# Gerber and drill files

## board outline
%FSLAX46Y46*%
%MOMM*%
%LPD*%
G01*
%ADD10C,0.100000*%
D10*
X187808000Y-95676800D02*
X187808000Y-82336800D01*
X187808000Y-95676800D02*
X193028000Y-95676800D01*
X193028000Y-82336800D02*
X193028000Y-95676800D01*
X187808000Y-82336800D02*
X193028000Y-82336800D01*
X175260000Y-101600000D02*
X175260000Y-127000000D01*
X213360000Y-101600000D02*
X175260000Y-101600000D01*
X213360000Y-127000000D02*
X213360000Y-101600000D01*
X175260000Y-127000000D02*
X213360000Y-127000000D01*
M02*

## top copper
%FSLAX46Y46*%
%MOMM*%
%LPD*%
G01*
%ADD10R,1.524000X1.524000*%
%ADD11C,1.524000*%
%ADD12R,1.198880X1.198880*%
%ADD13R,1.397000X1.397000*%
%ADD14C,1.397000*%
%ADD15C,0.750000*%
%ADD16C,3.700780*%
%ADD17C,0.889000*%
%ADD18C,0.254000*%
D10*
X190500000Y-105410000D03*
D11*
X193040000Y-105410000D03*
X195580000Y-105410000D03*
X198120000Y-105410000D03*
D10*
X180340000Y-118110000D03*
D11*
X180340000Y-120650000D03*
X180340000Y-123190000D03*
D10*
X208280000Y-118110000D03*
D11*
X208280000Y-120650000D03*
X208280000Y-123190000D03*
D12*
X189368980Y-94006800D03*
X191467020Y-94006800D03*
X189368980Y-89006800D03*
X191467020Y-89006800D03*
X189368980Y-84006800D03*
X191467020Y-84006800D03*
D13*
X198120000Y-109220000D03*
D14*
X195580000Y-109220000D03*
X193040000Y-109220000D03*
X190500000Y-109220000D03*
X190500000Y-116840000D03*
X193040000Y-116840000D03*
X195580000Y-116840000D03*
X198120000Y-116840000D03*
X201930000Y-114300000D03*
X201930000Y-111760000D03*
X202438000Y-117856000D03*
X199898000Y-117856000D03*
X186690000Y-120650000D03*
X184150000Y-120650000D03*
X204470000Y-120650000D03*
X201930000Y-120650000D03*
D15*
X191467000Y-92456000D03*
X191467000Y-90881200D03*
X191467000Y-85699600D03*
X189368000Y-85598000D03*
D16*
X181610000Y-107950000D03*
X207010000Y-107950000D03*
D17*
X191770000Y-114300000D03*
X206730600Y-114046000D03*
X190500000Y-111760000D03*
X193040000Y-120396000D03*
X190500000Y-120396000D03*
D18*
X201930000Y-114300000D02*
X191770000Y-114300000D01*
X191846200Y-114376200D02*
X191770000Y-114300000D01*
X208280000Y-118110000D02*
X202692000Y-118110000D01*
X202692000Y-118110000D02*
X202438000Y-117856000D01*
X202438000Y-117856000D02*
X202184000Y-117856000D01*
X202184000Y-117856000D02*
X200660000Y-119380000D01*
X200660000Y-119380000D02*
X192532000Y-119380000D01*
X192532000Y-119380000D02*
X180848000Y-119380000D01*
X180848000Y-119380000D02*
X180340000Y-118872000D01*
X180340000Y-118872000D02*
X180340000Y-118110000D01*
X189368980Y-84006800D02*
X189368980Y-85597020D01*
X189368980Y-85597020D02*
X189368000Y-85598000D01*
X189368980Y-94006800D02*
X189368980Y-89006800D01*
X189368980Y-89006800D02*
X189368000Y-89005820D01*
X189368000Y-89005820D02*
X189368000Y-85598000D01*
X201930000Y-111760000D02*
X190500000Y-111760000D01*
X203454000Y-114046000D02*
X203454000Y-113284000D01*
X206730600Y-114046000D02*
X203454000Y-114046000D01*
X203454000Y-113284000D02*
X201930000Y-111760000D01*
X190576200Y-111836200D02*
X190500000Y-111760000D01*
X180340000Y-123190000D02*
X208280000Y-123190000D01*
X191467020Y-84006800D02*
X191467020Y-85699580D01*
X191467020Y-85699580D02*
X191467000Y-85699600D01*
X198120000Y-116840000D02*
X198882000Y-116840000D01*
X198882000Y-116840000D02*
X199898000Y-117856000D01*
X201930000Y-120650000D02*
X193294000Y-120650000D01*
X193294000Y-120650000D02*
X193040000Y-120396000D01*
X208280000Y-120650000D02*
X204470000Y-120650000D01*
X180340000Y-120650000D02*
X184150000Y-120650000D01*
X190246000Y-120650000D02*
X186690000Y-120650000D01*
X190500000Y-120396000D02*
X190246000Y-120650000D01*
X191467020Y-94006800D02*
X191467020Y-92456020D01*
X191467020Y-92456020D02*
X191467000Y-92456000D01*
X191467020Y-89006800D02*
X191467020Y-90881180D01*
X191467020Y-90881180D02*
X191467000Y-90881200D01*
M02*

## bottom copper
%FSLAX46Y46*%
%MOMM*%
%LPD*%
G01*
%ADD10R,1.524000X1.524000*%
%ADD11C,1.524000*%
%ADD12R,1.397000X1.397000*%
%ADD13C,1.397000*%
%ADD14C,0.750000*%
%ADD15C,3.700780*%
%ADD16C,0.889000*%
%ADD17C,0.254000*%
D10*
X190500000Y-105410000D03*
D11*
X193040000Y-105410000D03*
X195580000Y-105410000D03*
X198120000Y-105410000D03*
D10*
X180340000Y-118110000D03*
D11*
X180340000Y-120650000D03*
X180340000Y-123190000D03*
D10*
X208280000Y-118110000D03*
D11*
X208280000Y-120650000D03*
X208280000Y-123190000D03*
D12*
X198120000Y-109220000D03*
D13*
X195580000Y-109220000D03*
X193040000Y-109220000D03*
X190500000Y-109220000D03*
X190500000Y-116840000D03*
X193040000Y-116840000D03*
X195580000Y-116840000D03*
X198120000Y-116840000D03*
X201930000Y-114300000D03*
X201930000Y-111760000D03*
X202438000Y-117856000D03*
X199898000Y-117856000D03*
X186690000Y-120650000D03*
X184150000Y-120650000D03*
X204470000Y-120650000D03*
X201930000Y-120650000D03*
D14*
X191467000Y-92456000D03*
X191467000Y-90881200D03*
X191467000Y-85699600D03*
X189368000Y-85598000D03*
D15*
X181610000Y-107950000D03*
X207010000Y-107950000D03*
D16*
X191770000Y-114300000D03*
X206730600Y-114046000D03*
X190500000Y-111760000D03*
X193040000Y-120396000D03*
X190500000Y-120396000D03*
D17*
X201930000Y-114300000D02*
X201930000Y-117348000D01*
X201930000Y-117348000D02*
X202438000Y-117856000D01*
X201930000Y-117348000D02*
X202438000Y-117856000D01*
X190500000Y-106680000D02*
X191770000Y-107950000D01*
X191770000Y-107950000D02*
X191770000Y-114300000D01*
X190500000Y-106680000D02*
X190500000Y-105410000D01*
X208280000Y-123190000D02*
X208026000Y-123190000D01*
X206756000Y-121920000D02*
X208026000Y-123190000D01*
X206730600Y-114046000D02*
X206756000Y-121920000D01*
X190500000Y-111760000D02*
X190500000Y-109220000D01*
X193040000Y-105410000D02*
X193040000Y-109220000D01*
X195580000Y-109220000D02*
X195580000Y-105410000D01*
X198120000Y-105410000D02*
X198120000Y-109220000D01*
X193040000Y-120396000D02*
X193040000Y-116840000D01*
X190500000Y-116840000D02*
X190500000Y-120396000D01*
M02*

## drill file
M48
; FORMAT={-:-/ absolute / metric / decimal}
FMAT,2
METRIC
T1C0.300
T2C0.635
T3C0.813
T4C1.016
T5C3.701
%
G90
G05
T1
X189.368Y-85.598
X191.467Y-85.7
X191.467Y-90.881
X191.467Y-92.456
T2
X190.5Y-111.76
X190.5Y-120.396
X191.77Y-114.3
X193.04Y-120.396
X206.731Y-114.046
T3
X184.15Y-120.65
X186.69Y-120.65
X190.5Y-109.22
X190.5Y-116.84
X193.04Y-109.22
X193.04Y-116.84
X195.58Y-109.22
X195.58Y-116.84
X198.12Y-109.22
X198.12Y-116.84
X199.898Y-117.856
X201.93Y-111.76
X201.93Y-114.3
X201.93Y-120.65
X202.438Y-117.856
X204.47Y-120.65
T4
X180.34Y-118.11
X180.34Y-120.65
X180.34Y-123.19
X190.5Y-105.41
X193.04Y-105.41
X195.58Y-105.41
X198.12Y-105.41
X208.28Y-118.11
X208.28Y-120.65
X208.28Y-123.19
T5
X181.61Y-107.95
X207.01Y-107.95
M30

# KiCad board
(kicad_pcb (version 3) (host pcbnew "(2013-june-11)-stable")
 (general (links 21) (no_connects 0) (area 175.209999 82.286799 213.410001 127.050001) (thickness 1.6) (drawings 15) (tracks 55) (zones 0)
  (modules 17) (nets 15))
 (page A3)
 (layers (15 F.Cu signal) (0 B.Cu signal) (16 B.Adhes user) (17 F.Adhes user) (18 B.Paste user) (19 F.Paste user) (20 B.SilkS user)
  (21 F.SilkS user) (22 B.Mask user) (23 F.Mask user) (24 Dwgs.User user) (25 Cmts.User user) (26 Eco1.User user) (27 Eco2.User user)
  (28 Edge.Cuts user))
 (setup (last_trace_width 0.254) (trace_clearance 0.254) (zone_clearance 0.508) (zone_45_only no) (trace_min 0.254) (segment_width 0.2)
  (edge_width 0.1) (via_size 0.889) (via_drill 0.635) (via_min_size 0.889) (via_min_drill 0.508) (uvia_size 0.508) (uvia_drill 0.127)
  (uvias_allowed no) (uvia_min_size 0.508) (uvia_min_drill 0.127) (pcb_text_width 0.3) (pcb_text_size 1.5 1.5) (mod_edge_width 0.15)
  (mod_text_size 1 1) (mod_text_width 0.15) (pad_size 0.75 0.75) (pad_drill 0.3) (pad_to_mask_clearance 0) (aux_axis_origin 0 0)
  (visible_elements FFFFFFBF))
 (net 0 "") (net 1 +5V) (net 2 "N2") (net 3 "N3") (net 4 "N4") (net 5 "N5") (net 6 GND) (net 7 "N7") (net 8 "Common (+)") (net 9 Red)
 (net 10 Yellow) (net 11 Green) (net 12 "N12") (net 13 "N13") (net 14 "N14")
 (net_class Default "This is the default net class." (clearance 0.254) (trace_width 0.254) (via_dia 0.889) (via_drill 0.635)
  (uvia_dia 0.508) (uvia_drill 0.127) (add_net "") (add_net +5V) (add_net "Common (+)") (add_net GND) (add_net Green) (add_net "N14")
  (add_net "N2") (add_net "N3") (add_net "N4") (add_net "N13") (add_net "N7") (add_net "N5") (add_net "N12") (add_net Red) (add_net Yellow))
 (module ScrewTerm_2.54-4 (layer F.Cu) (at 194.31 105.41)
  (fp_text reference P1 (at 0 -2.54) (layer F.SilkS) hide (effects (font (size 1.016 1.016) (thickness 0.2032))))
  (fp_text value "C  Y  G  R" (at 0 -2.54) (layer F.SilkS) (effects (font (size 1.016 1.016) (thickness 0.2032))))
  (pad 1 thru_hole rect (at -3.81 0) (size 1.524 1.524) (drill 1.016) (layers *.Cu *.Mask F.SilkS) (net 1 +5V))
  (pad 2 thru_hole circle (at -1.27 0) (size 1.524 1.524) (drill 1.016) (layers *.Cu *.Mask F.SilkS) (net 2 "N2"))
  (pad 3 thru_hole circle (at 1.27 0) (size 1.524 1.524) (drill 1.016) (layers *.Cu *.Mask F.SilkS) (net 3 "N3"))
  (pad 4 thru_hole circle (at 3.81 0) (size 1.524 1.524) (drill 1.016) (layers *.Cu *.Mask F.SilkS) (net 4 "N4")))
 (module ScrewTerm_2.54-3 (layer F.Cu) (at 180.34 120.65 270)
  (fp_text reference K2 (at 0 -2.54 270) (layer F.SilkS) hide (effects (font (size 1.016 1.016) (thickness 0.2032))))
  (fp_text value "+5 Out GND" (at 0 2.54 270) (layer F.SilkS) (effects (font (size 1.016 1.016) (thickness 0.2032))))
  (pad 1 thru_hole rect (at -2.54 0 270) (size 1.524 1.524) (drill 1.016) (layers *.Cu *.Mask F.SilkS) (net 1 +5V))
  (pad 2 thru_hole circle (at 0 0 270) (size 1.524 1.524) (drill 1.016) (layers *.Cu *.Mask F.SilkS) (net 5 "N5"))
  (pad 3 thru_hole circle (at 2.54 0 270) (size 1.524 1.524) (drill 1.016) (layers *.Cu *.Mask F.SilkS) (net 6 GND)))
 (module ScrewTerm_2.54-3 (layer F.Cu) (at 208.28 120.65 270)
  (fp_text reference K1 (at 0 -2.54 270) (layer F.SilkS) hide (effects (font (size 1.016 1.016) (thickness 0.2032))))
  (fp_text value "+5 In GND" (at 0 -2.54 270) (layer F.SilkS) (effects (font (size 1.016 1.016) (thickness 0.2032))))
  (pad 1 thru_hole rect (at -2.54 0 270) (size 1.524 1.524) (drill 1.016) (layers *.Cu *.Mask F.SilkS) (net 1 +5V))
  (pad 2 thru_hole circle (at 0 0 270) (size 1.524 1.524) (drill 1.016) (layers *.Cu *.Mask F.SilkS) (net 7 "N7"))
  (pad 3 thru_hole circle (at 2.54 0 270) (size 1.524 1.524) (drill 1.016) (layers *.Cu *.Mask F.SilkS) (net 6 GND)))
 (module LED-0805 (layer F.Cu) (at 190.418 94.0068)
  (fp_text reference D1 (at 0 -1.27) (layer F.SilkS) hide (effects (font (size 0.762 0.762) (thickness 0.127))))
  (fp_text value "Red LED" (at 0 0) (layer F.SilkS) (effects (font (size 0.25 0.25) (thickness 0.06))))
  (pad 1 smd rect (at -1.04902 0) (size 1.19888 1.19888) (layers F.Cu F.Paste F.Mask) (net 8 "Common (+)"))
  (pad 2 smd rect (at 1.04902 0) (size 1.19888 1.19888) (layers F.Cu F.Paste F.Mask) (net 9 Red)))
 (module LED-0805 (layer F.Cu) (at 190.418 89.0068)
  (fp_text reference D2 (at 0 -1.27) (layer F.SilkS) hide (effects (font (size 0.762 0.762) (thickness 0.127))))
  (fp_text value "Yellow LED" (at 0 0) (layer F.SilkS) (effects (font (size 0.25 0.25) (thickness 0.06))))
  (pad 1 smd rect (at -1.04902 0) (size 1.19888 1.19888) (layers F.Cu F.Paste F.Mask) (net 8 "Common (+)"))
  (pad 2 smd rect (at 1.04902 0) (size 1.19888 1.19888) (layers F.Cu F.Paste F.Mask) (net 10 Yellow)))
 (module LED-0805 (layer F.Cu) (at 190.418 84.0068)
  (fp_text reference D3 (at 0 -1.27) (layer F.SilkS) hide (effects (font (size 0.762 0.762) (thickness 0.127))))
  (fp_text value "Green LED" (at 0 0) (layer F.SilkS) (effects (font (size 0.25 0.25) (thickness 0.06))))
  (pad 1 smd rect (at -1.04902 0) (size 1.19888 1.19888) (layers F.Cu F.Paste F.Mask) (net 8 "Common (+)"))
  (pad 2 smd rect (at 1.04902 0) (size 1.19888 1.19888) (layers F.Cu F.Paste F.Mask) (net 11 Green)))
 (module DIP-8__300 (layer F.Cu) (at 194.31 113.03 180)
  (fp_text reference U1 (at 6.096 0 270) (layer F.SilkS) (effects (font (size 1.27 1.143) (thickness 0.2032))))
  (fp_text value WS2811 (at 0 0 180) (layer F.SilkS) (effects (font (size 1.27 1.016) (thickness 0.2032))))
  (pad 1 thru_hole rect (at -3.81 3.81 180) (size 1.397 1.397) (drill 0.8128) (layers *.Cu *.Mask F.SilkS) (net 4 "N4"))
  (pad 2 thru_hole circle (at -1.27 3.81 180) (size 1.397 1.397) (drill 0.8128) (layers *.Cu *.Mask F.SilkS) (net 3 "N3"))
  (pad 3 thru_hole circle (at 1.27 3.81 180) (size 1.397 1.397) (drill 0.8128) (layers *.Cu *.Mask F.SilkS) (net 2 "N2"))
  (pad 4 thru_hole circle (at 3.81 3.81 180) (size 1.397 1.397) (drill 0.8128) (layers *.Cu *.Mask F.SilkS) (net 6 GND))
  (pad 5 thru_hole circle (at 3.81 -3.81 180) (size 1.397 1.397) (drill 0.8128) (layers *.Cu *.Mask F.SilkS) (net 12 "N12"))
  (pad 6 thru_hole circle (at 1.27 -3.81 180) (size 1.397 1.397) (drill 0.8128) (layers *.Cu *.Mask F.SilkS) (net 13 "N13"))
  (pad 7 thru_hole circle (at -1.27 -3.81 180) (size 1.397 1.397) (drill 0.8128) (layers *.Cu *.Mask F.SilkS))
  (pad 8 thru_hole circle (at -3.81 -3.81 180) (size 1.397 1.397) (drill 0.8128) (layers *.Cu *.Mask F.SilkS) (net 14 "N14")))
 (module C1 (layer F.Cu) (at 201.93 113.03 90)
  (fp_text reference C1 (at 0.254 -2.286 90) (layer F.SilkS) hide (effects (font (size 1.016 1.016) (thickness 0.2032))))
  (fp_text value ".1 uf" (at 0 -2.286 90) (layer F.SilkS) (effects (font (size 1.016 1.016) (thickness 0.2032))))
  (pad 1 thru_hole circle (at -1.27 0 90) (size 1.397 1.397) (drill 0.8128) (layers *.Cu *.Mask F.SilkS) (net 1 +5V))
  (pad 2 thru_hole circle (at 1.27 0 90) (size 1.397 1.397) (drill 0.8128) (layers *.Cu *.Mask F.SilkS) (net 6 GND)))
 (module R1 (layer F.Cu) (at 201.168 117.856 180) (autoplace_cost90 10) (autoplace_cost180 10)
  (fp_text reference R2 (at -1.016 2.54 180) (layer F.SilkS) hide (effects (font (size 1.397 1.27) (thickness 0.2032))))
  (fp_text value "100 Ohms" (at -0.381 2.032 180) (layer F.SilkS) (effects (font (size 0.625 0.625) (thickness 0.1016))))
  (pad 1 thru_hole circle (at -1.27 0 180) (size 1.397 1.397) (drill 0.8128) (layers *.Cu *.Mask F.SilkS) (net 1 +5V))
  (pad 2 thru_hole circle (at 1.27 0 180) (size 1.397 1.397) (drill 0.8128) (layers *.Cu *.Mask F.SilkS) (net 14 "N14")))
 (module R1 (layer F.Cu) (at 185.42 120.65 180) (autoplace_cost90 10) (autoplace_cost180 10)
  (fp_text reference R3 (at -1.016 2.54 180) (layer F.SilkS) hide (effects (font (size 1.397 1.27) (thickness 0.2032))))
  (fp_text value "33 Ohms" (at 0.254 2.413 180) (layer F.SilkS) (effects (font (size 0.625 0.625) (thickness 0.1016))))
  (pad 1 thru_hole circle (at -1.27 0 180) (size 1.397 1.397) (drill 0.8128) (layers *.Cu *.Mask F.SilkS) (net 12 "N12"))
  (pad 2 thru_hole circle (at 1.27 0 180) (size 1.397 1.397) (drill 0.8128) (layers *.Cu *.Mask F.SilkS) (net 5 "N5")))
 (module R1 (layer F.Cu) (at 203.2 120.65 180) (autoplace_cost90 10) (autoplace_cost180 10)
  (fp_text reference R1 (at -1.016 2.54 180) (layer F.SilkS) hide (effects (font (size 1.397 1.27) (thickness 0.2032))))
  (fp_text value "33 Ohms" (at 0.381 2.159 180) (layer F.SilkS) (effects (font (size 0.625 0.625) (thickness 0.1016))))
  (pad 1 thru_hole circle (at -1.27 0 180) (size 1.397 1.397) (drill 0.8128) (layers *.Cu *.Mask F.SilkS) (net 7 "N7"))
  (pad 2 thru_hole circle (at 1.27 0 180) (size 1.397 1.397) (drill 0.8128) (layers *.Cu *.Mask F.SilkS) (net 13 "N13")))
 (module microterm (layer F.Cu) (at 191.467 92.456)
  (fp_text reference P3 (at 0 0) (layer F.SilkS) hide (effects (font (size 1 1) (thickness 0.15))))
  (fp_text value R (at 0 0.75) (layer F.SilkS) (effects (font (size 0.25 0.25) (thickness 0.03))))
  (pad 1 thru_hole circle (at 0 0) (size 0.75 0.75) (drill 0.3) (layers *.Cu *.Mask F.SilkS) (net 9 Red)))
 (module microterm (layer F.Cu) (at 191.467 90.8812)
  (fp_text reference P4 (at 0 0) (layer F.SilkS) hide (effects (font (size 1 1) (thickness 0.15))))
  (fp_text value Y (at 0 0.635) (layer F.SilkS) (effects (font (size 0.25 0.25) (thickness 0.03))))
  (pad 1 thru_hole circle (at 0 0) (size 0.75 0.75) (drill 0.3) (layers *.Cu *.Mask F.SilkS) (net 10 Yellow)))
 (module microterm (layer F.Cu) (at 191.467 85.6996)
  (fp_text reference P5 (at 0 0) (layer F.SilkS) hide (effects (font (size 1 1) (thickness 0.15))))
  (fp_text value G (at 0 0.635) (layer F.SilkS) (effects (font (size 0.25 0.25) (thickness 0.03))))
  (pad 1 thru_hole circle (at 0 0) (size 0.75 0.75) (drill 0.3) (layers *.Cu *.Mask F.SilkS) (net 11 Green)))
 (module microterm (layer F.Cu) (at 189.368 85.598)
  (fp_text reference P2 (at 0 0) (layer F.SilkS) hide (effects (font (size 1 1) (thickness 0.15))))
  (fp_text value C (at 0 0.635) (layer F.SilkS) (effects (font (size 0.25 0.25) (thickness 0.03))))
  (pad 1 thru_hole circle (at 0 0) (size 0.75 0.75) (drill 0.3) (layers *.Cu *.Mask F.SilkS) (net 8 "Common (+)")))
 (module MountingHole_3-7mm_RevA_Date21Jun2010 (layer F.Cu) (at 181.61 107.95)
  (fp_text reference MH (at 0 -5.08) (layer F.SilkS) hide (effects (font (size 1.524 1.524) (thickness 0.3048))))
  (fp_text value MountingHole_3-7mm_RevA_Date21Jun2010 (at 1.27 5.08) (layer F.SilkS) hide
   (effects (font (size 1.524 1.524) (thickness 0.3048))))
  (pad 1 thru_hole circle (at 0 0) (size 3.70078 3.70078) (drill 3.70078) (layers)))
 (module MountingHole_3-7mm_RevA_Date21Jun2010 (layer F.Cu) (at 207.01 107.95)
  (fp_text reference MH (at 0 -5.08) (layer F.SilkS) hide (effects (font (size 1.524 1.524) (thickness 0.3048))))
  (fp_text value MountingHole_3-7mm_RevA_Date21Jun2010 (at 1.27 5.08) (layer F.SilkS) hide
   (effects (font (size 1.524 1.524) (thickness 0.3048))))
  (pad 1 thru_hole circle (at 0 0) (size 3.70078 3.70078) (drill 3.70078) (layers)))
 (gr_line (start 187.808 95.6768) (end 187.808 82.3368) (angle 90) (layer Edge.Cuts) (width 0.1))
 (gr_line (start 187.808 95.6768) (end 193.028 95.6768) (angle 90) (layer Edge.Cuts) (width 0.1))
 (gr_line (start 193.028 82.3368) (end 193.028 95.6768) (angle 90) (layer Edge.Cuts) (width 0.1))
 (gr_line (start 187.808 82.3368) (end 193.028 82.3368) (angle 90) (layer Edge.Cuts) (width 0.1))
 (gr_line (start 175.26 101.6) (end 175.26 127) (angle 90) (layer Edge.Cuts) (width 0.1))
 (gr_line (start 213.36 101.6) (end 175.26 101.6) (angle 90) (layer Edge.Cuts) (width 0.1))
 (gr_line (start 213.36 127) (end 213.36 101.6) (angle 90) (layer Edge.Cuts) (width 0.1))
 (gr_line (start 175.26 127) (end 213.36 127) (angle 90) (layer Edge.Cuts) (width 0.1))
 (segment (start 201.93 114.3) (end 201.93 117.348) (width 0.254) (layer B.Cu) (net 1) (status 400000))
 (segment (start 201.93 117.348) (end 202.438 117.856) (width 0.254) (layer B.Cu) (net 1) (status 800000))
 (segment (start 201.93 114.3) (end 191.77 114.3) (width 0.254) (layer F.Cu) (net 1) (status 400000))
 (segment (start 201.93 117.348) (end 202.438 117.856) (width 0.254) (layer B.Cu) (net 1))
 (segment (start 190.5 106.68) (end 191.77 107.95) (width 0.254) (layer B.Cu) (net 1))
 (segment (start 191.77 107.95) (end 191.77 114.3) (width 0.254) (layer B.Cu) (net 1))
 (via (at 191.77 114.3) (size 0.889) (layers F.Cu B.Cu) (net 1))
 (segment (start 190.5 106.68) (end 190.5 105.41) (width 0.254) (layer B.Cu) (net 1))
 (segment (start 191.8462 114.3762) (end 191.77 114.3) (width 0.254) (layer F.Cu) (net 1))
 (segment (start 208.28 118.11) (end 202.692 118.11) (width 0.254) (layer F.Cu) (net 1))
 (segment (start 202.692 118.11) (end 202.438 117.856) (width 0.254) (layer F.Cu) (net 1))
 (segment (start 202.438 117.856) (end 202.184 117.856) (width 0.254) (layer F.Cu) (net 1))
 (segment (start 202.184 117.856) (end 200.66 119.38) (width 0.254) (layer F.Cu) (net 1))
 (segment (start 200.66 119.38) (end 192.532 119.38) (width 0.254) (layer F.Cu) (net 1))
 (segment (start 192.532 119.38) (end 180.848 119.38) (width 0.254) (layer F.Cu) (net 1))
 (segment (start 180.848 119.38) (end 180.34 118.872) (width 0.254) (layer F.Cu) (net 1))
 (segment (start 180.34 118.872) (end 180.34 118.11) (width 0.254) (layer F.Cu) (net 1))
 (segment (start 189.36898 84.0068) (end 189.36898 85.59702) (width 0.254) (layer F.Cu) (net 8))
 (segment (start 189.36898 85.59702) (end 189.368 85.598) (width 0.254) (layer F.Cu) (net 8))
 (segment (start 189.36898 94.0068) (end 189.36898 89.0068) (width 0.254) (layer F.Cu) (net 8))
 (segment (start 189.36898 89.0068) (end 189.368 89.00582) (width 0.254) (layer F.Cu) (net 8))
 (segment (start 189.368 89.00582) (end 189.368 85.598) (width 0.254) (layer F.Cu) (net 8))
 (segment (start 201.93 111.76) (end 190.5 111.76) (width 0.254) (layer F.Cu) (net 6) (status 400000))
 (segment (start 203.454 114.046) (end 203.454 113.284) (width 0.254) (layer F.Cu) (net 6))
 (segment (start 208.28 123.19) (end 208.026 123.19) (width 0.254) (layer B.Cu) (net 6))
 (segment (start 206.756 121.92) (end 208.026 123.19) (width 0.254) (layer B.Cu) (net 6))
 (segment (start 206.7306 114.046) (end 206.756 121.92) (width 0.254) (layer B.Cu) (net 6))
 (via (at 206.7306 114.046) (size 0.889) (layers F.Cu B.Cu) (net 6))
 (segment (start 206.7306 114.046) (end 203.454 114.046) (width 0.254) (layer F.Cu) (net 6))
 (segment (start 203.454 113.284) (end 201.93 111.76) (width 0.254) (layer F.Cu) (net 6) (status 800000))
 (via (at 190.5 111.76) (size 0.889) (layers F.Cu B.Cu) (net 6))
 (segment (start 190.5 111.76) (end 190.5 109.22) (width 0.254) (layer B.Cu) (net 6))
 (segment (start 190.5762 111.8362) (end 190.5 111.76) (width 0.254) (layer F.Cu) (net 6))
 (segment (start 180.34 123.19) (end 208.28 123.19) (width 0.254) (layer F.Cu) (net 6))
 (segment (start 191.46702 84.0068) (end 191.46702 85.69958) (width 0.254) (layer F.Cu) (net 11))
 (segment (start 191.46702 85.69958) (end 191.467 85.6996) (width 0.254) (layer F.Cu) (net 11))
 (segment (start 198.12 116.84) (end 198.882 116.84) (width 0.254) (layer F.Cu) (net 14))
 (segment (start 198.882 116.84) (end 199.898 117.856) (width 0.254) (layer F.Cu) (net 14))
 (segment (start 193.04 105.41) (end 193.04 109.22) (width 0.254) (layer B.Cu) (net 2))
 (segment (start 195.58 109.22) (end 195.58 105.41) (width 0.254) (layer B.Cu) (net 3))
 (segment (start 198.12 105.41) (end 198.12 109.22) (width 0.254) (layer B.Cu) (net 4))
 (segment (start 201.93 120.65) (end 193.294 120.65) (width 0.254) (layer F.Cu) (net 13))
 (segment (start 193.04 120.396) (end 193.04 116.84) (width 0.254) (layer B.Cu) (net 13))
 (via (at 193.04 120.396) (size 0.889) (layers F.Cu B.Cu) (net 13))
 (segment (start 193.294 120.65) (end 193.04 120.396) (width 0.254) (layer F.Cu) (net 13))
 (segment (start 208.28 120.65) (end 204.47 120.65) (width 0.254) (layer F.Cu) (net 7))
 (segment (start 180.34 120.65) (end 184.15 120.65) (width 0.254) (layer F.Cu) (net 5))
 (segment (start 190.5 116.84) (end 190.5 120.396) (width 0.254) (layer B.Cu) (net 12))
 (segment (start 190.246 120.65) (end 186.69 120.65) (width 0.254) (layer F.Cu) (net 12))
 (segment (start 190.5 120.396) (end 190.246 120.65) (width 0.254) (layer F.Cu) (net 12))
 (via (at 190.5 120.396) (size 0.889) (layers F.Cu B.Cu) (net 12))
 (segment (start 191.46702 94.0068) (end 191.46702 92.45602) (width 0.254) (layer F.Cu) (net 9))
 (segment (start 191.46702 92.45602) (end 191.467 92.456) (width 0.254) (layer F.Cu) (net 9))
 (segment (start 191.46702 89.0068) (end 191.46702 90.88118) (width 0.254) (layer F.Cu) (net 10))
 (segment (start 191.46702 90.88118) (end 191.467 90.8812) (width 0.254) (layer F.Cu) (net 10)))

